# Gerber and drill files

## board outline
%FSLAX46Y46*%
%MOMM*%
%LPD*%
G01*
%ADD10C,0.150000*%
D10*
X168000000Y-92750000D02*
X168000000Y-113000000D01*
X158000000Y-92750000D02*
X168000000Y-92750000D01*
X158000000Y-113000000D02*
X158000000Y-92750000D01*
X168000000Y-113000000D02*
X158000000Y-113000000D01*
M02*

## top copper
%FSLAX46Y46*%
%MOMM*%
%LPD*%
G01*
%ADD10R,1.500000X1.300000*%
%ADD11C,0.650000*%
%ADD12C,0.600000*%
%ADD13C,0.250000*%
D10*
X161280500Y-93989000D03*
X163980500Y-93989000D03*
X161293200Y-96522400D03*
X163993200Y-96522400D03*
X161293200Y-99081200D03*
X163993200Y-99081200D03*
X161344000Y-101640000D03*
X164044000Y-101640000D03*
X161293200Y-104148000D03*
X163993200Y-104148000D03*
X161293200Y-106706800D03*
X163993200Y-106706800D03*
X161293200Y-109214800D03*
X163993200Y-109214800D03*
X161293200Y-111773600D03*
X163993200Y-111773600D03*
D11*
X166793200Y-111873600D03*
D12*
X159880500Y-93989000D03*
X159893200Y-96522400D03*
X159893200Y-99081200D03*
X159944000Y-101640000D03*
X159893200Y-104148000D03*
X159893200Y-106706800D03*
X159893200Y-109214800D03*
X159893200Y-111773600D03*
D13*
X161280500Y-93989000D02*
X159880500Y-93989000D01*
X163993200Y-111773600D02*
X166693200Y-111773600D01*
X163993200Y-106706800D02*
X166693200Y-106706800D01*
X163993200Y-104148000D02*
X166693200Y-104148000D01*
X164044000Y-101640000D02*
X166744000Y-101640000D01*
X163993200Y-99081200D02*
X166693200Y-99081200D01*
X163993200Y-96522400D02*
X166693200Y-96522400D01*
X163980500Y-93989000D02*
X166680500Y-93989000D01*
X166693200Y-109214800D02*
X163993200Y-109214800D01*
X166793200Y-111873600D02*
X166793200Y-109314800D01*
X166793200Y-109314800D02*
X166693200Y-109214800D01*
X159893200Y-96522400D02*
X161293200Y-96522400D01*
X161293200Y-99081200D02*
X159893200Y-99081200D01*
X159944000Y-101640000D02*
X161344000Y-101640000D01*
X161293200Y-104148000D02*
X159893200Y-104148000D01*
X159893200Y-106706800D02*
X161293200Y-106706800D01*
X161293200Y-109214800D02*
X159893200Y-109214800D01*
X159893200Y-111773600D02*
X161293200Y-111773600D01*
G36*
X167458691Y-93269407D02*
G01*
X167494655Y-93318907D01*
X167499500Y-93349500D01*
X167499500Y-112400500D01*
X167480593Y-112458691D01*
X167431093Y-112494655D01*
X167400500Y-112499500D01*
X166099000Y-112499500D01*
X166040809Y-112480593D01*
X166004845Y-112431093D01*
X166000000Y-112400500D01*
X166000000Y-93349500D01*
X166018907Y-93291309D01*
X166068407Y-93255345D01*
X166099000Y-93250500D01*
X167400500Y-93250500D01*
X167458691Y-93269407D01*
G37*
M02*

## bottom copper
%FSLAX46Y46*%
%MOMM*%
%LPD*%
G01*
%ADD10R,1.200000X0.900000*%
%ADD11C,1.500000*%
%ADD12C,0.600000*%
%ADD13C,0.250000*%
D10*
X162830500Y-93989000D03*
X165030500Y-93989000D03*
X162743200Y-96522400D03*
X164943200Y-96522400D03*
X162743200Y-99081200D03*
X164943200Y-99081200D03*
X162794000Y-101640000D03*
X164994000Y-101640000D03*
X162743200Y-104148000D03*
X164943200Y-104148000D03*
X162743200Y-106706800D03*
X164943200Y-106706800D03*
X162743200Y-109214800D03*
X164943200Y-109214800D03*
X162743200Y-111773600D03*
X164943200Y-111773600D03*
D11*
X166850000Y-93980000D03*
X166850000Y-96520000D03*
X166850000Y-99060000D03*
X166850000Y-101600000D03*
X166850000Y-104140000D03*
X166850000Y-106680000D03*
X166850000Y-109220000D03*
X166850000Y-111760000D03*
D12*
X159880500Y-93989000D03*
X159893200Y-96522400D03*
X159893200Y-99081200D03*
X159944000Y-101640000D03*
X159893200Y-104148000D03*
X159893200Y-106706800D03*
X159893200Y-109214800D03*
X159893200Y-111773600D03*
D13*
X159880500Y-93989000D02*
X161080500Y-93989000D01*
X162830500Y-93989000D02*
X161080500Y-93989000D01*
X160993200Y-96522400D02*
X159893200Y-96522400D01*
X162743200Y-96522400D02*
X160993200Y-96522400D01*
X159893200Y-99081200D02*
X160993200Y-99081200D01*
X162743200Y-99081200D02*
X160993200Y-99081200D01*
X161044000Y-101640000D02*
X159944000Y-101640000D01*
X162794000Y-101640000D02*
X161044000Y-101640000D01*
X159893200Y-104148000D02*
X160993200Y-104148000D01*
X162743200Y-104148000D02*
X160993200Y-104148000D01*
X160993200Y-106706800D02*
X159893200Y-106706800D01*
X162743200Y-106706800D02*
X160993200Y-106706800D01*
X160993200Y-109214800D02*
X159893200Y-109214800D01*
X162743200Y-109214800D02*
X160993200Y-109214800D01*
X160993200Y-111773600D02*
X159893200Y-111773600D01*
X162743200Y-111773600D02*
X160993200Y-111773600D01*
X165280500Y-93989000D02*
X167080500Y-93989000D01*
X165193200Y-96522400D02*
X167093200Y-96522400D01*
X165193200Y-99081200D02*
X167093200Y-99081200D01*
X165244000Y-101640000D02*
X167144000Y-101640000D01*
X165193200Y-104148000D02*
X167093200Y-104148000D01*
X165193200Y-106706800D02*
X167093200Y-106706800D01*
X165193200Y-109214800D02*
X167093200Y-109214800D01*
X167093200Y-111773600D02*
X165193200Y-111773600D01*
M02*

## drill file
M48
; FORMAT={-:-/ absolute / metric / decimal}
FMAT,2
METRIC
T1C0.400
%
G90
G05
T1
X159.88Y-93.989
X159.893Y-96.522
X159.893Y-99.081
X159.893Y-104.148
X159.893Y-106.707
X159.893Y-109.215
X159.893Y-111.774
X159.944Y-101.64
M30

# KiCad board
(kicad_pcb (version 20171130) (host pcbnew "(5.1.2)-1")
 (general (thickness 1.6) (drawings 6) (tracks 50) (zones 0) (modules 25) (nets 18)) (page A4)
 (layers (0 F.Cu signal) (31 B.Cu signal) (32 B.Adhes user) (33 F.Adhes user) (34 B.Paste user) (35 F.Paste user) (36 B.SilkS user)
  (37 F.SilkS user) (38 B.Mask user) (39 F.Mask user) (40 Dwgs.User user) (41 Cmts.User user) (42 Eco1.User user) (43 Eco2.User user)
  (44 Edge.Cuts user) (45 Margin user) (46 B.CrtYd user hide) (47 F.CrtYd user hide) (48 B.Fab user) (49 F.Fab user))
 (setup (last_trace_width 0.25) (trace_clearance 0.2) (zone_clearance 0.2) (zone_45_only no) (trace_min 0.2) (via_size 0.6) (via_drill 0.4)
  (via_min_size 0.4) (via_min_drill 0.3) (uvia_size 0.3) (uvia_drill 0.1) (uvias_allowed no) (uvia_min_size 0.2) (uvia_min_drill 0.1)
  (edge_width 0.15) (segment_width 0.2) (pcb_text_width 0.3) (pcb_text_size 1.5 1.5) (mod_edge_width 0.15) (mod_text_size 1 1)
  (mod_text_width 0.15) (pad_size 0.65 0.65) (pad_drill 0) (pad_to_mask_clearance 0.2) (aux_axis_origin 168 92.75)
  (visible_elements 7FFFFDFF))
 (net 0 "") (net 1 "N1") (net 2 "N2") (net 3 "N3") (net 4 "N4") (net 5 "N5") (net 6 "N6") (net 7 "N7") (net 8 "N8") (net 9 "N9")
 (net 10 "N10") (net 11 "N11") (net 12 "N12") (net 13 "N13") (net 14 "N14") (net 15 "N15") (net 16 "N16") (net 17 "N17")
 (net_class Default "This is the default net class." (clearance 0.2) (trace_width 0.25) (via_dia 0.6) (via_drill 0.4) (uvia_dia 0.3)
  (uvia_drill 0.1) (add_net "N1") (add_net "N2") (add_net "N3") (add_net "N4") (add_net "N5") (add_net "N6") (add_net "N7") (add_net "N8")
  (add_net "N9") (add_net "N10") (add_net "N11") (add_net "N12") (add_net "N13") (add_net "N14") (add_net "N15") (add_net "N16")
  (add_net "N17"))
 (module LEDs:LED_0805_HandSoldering (layer F.Cu) (at 162.6305 93.989)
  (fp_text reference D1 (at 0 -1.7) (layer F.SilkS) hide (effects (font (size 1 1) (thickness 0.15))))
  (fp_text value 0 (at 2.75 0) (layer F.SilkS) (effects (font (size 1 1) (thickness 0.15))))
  (pad 1 smd rect (at -1.35 0) (size 1.5 1.3) (layers F.Cu F.Paste F.Mask) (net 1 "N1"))
  (pad 2 smd rect (at 1.35 0) (size 1.5 1.3) (layers F.Cu F.Paste F.Mask) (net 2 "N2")))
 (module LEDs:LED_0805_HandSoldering (layer F.Cu) (at 162.6432 96.5224)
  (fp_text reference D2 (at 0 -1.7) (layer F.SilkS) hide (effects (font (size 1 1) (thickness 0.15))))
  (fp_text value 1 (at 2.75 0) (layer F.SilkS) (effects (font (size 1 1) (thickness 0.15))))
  (pad 1 smd rect (at -1.35 0) (size 1.5 1.3) (layers F.Cu F.Paste F.Mask) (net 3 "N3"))
  (pad 2 smd rect (at 1.35 0) (size 1.5 1.3) (layers F.Cu F.Paste F.Mask) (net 2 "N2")))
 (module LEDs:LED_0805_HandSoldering (layer F.Cu) (at 162.6432 99.0812)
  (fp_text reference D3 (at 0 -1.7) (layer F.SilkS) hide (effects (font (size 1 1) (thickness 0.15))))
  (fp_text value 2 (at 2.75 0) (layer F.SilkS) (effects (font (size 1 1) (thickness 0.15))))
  (pad 1 smd rect (at -1.35 0) (size 1.5 1.3) (layers F.Cu F.Paste F.Mask) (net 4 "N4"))
  (pad 2 smd rect (at 1.35 0) (size 1.5 1.3) (layers F.Cu F.Paste F.Mask) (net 2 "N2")))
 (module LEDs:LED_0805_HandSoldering (layer F.Cu) (at 162.694 101.64)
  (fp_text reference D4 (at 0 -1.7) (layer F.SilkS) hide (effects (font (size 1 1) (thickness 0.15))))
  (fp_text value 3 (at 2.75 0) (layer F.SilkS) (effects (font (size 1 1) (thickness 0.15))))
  (pad 1 smd rect (at -1.35 0) (size 1.5 1.3) (layers F.Cu F.Paste F.Mask) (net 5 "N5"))
  (pad 2 smd rect (at 1.35 0) (size 1.5 1.3) (layers F.Cu F.Paste F.Mask) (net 2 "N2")))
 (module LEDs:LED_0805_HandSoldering (layer F.Cu) (at 162.6432 104.148)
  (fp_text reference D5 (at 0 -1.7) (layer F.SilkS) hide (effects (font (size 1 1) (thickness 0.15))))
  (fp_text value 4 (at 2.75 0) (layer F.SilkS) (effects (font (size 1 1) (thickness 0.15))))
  (pad 1 smd rect (at -1.35 0) (size 1.5 1.3) (layers F.Cu F.Paste F.Mask) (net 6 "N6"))
  (pad 2 smd rect (at 1.35 0) (size 1.5 1.3) (layers F.Cu F.Paste F.Mask) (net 2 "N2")))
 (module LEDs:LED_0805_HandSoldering (layer F.Cu) (at 162.6432 106.7068)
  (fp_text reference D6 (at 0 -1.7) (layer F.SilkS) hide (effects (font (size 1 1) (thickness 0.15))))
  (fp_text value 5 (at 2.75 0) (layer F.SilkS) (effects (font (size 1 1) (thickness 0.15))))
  (pad 1 smd rect (at -1.35 0) (size 1.5 1.3) (layers F.Cu F.Paste F.Mask) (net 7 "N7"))
  (pad 2 smd rect (at 1.35 0) (size 1.5 1.3) (layers F.Cu F.Paste F.Mask) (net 2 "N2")))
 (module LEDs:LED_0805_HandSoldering (layer F.Cu) (at 162.6432 109.2148)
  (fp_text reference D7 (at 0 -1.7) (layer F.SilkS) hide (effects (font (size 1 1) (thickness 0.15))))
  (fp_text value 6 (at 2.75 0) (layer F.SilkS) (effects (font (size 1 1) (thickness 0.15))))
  (pad 1 smd rect (at -1.35 0) (size 1.5 1.3) (layers F.Cu F.Paste F.Mask) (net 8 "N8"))
  (pad 2 smd rect (at 1.35 0) (size 1.5 1.3) (layers F.Cu F.Paste F.Mask) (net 2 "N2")))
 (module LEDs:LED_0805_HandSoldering (layer F.Cu) (at 162.6432 111.7736)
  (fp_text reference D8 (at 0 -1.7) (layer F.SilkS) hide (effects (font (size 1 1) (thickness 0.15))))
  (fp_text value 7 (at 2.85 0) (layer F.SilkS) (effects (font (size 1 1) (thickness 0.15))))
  (pad 1 smd rect (at -1.35 0) (size 1.5 1.3) (layers F.Cu F.Paste F.Mask) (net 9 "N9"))
  (pad 2 smd rect (at 1.35 0) (size 1.5 1.3) (layers F.Cu F.Paste F.Mask) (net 2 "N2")))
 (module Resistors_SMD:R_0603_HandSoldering (layer B.Cu) (at 163.9305 93.989)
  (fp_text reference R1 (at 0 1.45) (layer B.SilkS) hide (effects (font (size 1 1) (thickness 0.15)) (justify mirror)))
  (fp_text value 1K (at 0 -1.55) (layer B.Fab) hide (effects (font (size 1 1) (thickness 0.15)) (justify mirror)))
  (pad 1 smd rect (at -1.1 0) (size 1.2 0.9) (layers B.Cu B.Paste B.Mask) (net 1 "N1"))
  (pad 2 smd rect (at 1.1 0) (size 1.2 0.9) (layers B.Cu B.Paste B.Mask) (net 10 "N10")))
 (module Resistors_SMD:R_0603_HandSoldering (layer B.Cu) (at 163.8432 96.5224)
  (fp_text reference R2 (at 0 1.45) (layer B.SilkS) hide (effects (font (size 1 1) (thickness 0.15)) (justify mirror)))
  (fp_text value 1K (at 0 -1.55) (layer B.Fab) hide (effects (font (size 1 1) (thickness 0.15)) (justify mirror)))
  (pad 1 smd rect (at -1.1 0) (size 1.2 0.9) (layers B.Cu B.Paste B.Mask) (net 3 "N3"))
  (pad 2 smd rect (at 1.1 0) (size 1.2 0.9) (layers B.Cu B.Paste B.Mask) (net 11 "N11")))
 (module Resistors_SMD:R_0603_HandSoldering (layer B.Cu) (at 163.8432 99.0812)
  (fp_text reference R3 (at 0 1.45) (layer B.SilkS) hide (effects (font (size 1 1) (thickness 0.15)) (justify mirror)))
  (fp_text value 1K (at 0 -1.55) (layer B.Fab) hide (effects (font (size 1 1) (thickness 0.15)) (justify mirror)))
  (pad 1 smd rect (at -1.1 0) (size 1.2 0.9) (layers B.Cu B.Paste B.Mask) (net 4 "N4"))
  (pad 2 smd rect (at 1.1 0) (size 1.2 0.9) (layers B.Cu B.Paste B.Mask) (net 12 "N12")))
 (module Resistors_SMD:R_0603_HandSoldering (layer B.Cu) (at 163.894 101.64)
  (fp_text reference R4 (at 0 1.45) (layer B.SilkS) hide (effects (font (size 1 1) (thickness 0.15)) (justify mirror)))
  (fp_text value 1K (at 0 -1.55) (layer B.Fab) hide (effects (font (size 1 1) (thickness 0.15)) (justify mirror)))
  (pad 1 smd rect (at -1.1 0) (size 1.2 0.9) (layers B.Cu B.Paste B.Mask) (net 5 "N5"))
  (pad 2 smd rect (at 1.1 0) (size 1.2 0.9) (layers B.Cu B.Paste B.Mask) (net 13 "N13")))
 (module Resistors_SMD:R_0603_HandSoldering (layer B.Cu) (at 163.8432 104.148)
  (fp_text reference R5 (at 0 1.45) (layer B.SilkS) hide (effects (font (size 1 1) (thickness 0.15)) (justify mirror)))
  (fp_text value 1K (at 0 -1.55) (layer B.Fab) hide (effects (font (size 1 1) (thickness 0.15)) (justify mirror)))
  (pad 1 smd rect (at -1.1 0) (size 1.2 0.9) (layers B.Cu B.Paste B.Mask) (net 6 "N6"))
  (pad 2 smd rect (at 1.1 0) (size 1.2 0.9) (layers B.Cu B.Paste B.Mask) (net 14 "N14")))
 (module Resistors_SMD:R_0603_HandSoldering (layer B.Cu) (at 163.8432 106.7068)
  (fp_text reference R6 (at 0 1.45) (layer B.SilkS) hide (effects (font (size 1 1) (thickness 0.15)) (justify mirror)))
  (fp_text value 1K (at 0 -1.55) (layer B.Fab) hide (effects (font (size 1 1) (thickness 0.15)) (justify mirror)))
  (pad 1 smd rect (at -1.1 0) (size 1.2 0.9) (layers B.Cu B.Paste B.Mask) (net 7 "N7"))
  (pad 2 smd rect (at 1.1 0) (size 1.2 0.9) (layers B.Cu B.Paste B.Mask) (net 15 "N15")))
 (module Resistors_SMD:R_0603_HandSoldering (layer B.Cu) (at 163.8432 109.2148)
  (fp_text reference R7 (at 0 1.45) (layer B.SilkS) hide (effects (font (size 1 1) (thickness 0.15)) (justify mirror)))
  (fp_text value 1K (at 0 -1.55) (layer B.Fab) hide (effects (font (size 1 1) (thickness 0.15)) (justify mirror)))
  (pad 1 smd rect (at -1.1 0) (size 1.2 0.9) (layers B.Cu B.Paste B.Mask) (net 8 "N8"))
  (pad 2 smd rect (at 1.1 0) (size 1.2 0.9) (layers B.Cu B.Paste B.Mask) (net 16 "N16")))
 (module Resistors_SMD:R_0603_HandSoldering (layer B.Cu) (at 163.8432 111.7736)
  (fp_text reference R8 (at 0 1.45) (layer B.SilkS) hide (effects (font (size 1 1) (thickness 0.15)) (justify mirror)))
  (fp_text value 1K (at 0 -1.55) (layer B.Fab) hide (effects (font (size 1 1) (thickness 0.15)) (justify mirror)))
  (pad 1 smd rect (at -1.1 0) (size 1.2 0.9) (layers B.Cu B.Paste B.Mask) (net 9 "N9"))
  (pad 2 smd rect (at 1.1 0) (size 1.2 0.9) (layers B.Cu B.Paste B.Mask) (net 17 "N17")))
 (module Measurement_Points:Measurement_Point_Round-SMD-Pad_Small (layer B.Cu) (at 166.85 93.98 180)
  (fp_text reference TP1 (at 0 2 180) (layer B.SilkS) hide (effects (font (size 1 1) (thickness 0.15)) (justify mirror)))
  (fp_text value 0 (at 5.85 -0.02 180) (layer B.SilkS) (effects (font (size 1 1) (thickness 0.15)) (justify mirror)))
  (pad 1 smd circle (at 0 0 180) (size 1.5 1.5) (layers B.Cu B.Mask) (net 10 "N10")))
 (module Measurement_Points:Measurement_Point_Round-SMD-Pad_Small (layer B.Cu) (at 166.85 96.52 180)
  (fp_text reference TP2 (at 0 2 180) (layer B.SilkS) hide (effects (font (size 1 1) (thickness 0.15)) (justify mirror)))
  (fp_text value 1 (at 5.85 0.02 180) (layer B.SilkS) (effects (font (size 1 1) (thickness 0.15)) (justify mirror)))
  (pad 1 smd circle (at 0 0 180) (size 1.5 1.5) (layers B.Cu B.Mask) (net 11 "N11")))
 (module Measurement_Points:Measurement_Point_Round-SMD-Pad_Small (layer B.Cu) (at 166.85 99.06 180)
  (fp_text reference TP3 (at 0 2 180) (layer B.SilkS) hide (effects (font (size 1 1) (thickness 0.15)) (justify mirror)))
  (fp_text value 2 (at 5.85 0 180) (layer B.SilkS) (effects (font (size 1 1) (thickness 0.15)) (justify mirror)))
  (pad 1 smd circle (at 0 0 180) (size 1.5 1.5) (layers B.Cu B.Mask) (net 12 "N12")))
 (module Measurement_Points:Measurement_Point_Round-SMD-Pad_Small (layer B.Cu) (at 166.85 101.6 180)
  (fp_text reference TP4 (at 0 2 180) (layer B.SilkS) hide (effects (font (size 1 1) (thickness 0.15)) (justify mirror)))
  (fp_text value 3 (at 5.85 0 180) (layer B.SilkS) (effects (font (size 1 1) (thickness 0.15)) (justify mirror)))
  (pad 1 smd circle (at 0 0 180) (size 1.5 1.5) (layers B.Cu B.Mask) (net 13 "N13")))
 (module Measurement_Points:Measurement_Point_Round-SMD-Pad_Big (layer F.Cu) (at 166.7932 111.8736)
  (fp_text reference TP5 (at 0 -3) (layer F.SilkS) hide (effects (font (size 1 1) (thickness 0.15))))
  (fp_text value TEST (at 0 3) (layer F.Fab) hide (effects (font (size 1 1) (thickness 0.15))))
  (pad 1 smd circle (at 0 0) (size 0.65 0.65) (layers F.Cu F.Mask) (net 2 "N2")))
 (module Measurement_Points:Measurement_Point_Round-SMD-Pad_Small (layer B.Cu) (at 166.85 104.14 180)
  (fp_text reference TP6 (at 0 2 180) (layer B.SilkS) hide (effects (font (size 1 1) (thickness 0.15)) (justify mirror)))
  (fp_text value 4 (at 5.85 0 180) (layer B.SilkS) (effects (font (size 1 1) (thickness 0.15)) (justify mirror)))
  (pad 1 smd circle (at 0 0 180) (size 1.5 1.5) (layers B.Cu B.Mask) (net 14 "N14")))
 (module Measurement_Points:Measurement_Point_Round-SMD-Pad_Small (layer B.Cu) (at 166.85 106.68 180)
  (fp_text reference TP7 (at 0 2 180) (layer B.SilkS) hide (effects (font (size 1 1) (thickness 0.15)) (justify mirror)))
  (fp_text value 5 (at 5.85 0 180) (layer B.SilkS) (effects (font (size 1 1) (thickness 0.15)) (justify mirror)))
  (pad 1 smd circle (at 0 0 180) (size 1.5 1.5) (layers B.Cu B.Mask) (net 15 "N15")))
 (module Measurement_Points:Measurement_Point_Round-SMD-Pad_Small (layer B.Cu) (at 166.85 109.22 180)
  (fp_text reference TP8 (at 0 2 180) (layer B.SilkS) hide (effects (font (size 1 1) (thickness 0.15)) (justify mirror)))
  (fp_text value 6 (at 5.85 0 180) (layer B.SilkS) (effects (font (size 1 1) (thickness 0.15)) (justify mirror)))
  (pad 1 smd circle (at 0 0 180) (size 1.5 1.5) (layers B.Cu B.Mask) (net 16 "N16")))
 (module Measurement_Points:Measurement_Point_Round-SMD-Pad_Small (layer B.Cu) (at 166.85 111.76 180)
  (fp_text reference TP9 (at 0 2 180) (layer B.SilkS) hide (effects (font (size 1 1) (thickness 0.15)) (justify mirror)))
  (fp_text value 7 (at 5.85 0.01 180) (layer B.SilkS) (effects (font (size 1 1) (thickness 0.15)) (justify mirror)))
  (pad 1 smd circle (at 0 0 180) (size 1.5 1.5) (layers B.Cu B.Mask) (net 17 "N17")))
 (gr_line (start 168 92.75) (end 168 113) (layer Edge.Cuts) (width 0.15))
 (gr_line (start 158 92.75) (end 168 92.75) (layer Edge.Cuts) (width 0.15))
 (gr_line (start 158 113) (end 158 92.75) (layer Edge.Cuts) (width 0.15))
 (gr_line (start 168 113) (end 158 113) (layer Edge.Cuts) (width 0.15))
 (segment (start 159.8805 93.989) (end 161.0805 93.989) (width 0.25) (layer B.Cu) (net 1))
 (segment (start 161.2805 93.989) (end 159.8805 93.989) (width 0.25) (layer F.Cu) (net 1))
 (via (at 159.8805 93.989) (size 0.6) (drill 0.4) (layers F.Cu B.Cu) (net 1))
 (segment (start 162.8305 93.989) (end 161.0805 93.989) (width 0.25) (layer B.Cu) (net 1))
 (segment (start 163.9932 111.7736) (end 166.6932 111.7736) (width 0.25) (layer F.Cu) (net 2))
 (segment (start 163.9932 106.7068) (end 166.6932 106.7068) (width 0.25) (layer F.Cu) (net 2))
 (segment (start 163.9932 104.148) (end 166.6932 104.148) (width 0.25) (layer F.Cu) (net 2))
 (segment (start 164.044 101.64) (end 166.744 101.64) (width 0.25) (layer F.Cu) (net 2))
 (segment (start 163.9932 99.0812) (end 166.6932 99.0812) (width 0.25) (layer F.Cu) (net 2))
 (segment (start 163.9932 96.5224) (end 166.6932 96.5224) (width 0.25) (layer F.Cu) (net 2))
 (segment (start 163.9805 93.989) (end 166.6805 93.989) (width 0.25) (layer F.Cu) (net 2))
 (segment (start 166.6932 109.2148) (end 163.9932 109.2148) (width 0.25) (layer F.Cu) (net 2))
 (segment (start 166.7932 111.8736) (end 166.7932 109.3148) (width 0.25) (layer F.Cu) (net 2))
 (segment (start 166.7932 109.3148) (end 166.6932 109.2148) (width 0.25) (layer F.Cu) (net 2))
 (segment (start 159.8932 96.5224) (end 161.2932 96.5224) (width 0.25) (layer F.Cu) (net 3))
 (segment (start 160.9932 96.5224) (end 159.8932 96.5224) (width 0.25) (layer B.Cu) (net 3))
 (via (at 159.8932 96.5224) (size 0.6) (drill 0.4) (layers F.Cu B.Cu) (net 3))
 (segment (start 162.7432 96.5224) (end 160.9932 96.5224) (width 0.25) (layer B.Cu) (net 3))
 (segment (start 159.8932 99.0812) (end 160.9932 99.0812) (width 0.25) (layer B.Cu) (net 4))
 (segment (start 161.2932 99.0812) (end 159.8932 99.0812) (width 0.25) (layer F.Cu) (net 4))
 (via (at 159.8932 99.0812) (size 0.6) (drill 0.4) (layers F.Cu B.Cu) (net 4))
 (segment (start 162.7432 99.0812) (end 160.9932 99.0812) (width 0.25) (layer B.Cu) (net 4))
 (segment (start 159.944 101.64) (end 161.344 101.64) (width 0.25) (layer F.Cu) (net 5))
 (segment (start 161.044 101.64) (end 159.944 101.64) (width 0.25) (layer B.Cu) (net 5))
 (via (at 159.944 101.64) (size 0.6) (drill 0.4) (layers F.Cu B.Cu) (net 5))
 (segment (start 162.794 101.64) (end 161.044 101.64) (width 0.25) (layer B.Cu) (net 5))
 (segment (start 159.8932 104.148) (end 160.9932 104.148) (width 0.25) (layer B.Cu) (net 6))
 (segment (start 161.2932 104.148) (end 159.8932 104.148) (width 0.25) (layer F.Cu) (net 6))
 (via (at 159.8932 104.148) (size 0.6) (drill 0.4) (layers F.Cu B.Cu) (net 6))
 (segment (start 162.7432 104.148) (end 160.9932 104.148) (width 0.25) (layer B.Cu) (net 6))
 (segment (start 159.8932 106.7068) (end 161.2932 106.7068) (width 0.25) (layer F.Cu) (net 7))
 (segment (start 160.9932 106.7068) (end 159.8932 106.7068) (width 0.25) (layer B.Cu) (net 7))
 (via (at 159.8932 106.7068) (size 0.6) (drill 0.4) (layers F.Cu B.Cu) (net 7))
 (segment (start 162.7432 106.7068) (end 160.9932 106.7068) (width 0.25) (layer B.Cu) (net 7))
 (segment (start 160.9932 109.2148) (end 159.8932 109.2148) (width 0.25) (layer B.Cu) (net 8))
 (segment (start 161.2932 109.2148) (end 159.8932 109.2148) (width 0.25) (layer F.Cu) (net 8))
 (via (at 159.8932 109.2148) (size 0.6) (drill 0.4) (layers F.Cu B.Cu) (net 8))
 (segment (start 162.7432 109.2148) (end 160.9932 109.2148) (width 0.25) (layer B.Cu) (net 8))
 (segment (start 159.8932 111.7736) (end 161.2932 111.7736) (width 0.25) (layer F.Cu) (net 9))
 (segment (start 160.9932 111.7736) (end 159.8932 111.7736) (width 0.25) (layer B.Cu) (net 9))
 (via (at 159.8932 111.7736) (size 0.6) (drill 0.4) (layers F.Cu B.Cu) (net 9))
 (segment (start 162.7432 111.7736) (end 160.9932 111.7736) (width 0.25) (layer B.Cu) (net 9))
 (segment (start 165.2805 93.989) (end 167.0805 93.989) (width 0.25) (layer B.Cu) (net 10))
 (segment (start 165.1932 96.5224) (end 167.0932 96.5224) (width 0.25) (layer B.Cu) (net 11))
 (segment (start 165.1932 99.0812) (end 167.0932 99.0812) (width 0.25) (layer B.Cu) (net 12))
 (segment (start 165.244 101.64) (end 167.144 101.64) (width 0.25) (layer B.Cu) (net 13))
 (segment (start 165.1932 104.148) (end 167.0932 104.148) (width 0.25) (layer B.Cu) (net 14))
 (segment (start 165.1932 106.7068) (end 167.0932 106.7068) (width 0.25) (layer B.Cu) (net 15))
 (segment (start 165.1932 109.2148) (end 167.0932 109.2148) (width 0.25) (layer B.Cu) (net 16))
 (segment (start 167.0932 111.7736) (end 165.1932 111.7736) (width 0.25) (layer B.Cu) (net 17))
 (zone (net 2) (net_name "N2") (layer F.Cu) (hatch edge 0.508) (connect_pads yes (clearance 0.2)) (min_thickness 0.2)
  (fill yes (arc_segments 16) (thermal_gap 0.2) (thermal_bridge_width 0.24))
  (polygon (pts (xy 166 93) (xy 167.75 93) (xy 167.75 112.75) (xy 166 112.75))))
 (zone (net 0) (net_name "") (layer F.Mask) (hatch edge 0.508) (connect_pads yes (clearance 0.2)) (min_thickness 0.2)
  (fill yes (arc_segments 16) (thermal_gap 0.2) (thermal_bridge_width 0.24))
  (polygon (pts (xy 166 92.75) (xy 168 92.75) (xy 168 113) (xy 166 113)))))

